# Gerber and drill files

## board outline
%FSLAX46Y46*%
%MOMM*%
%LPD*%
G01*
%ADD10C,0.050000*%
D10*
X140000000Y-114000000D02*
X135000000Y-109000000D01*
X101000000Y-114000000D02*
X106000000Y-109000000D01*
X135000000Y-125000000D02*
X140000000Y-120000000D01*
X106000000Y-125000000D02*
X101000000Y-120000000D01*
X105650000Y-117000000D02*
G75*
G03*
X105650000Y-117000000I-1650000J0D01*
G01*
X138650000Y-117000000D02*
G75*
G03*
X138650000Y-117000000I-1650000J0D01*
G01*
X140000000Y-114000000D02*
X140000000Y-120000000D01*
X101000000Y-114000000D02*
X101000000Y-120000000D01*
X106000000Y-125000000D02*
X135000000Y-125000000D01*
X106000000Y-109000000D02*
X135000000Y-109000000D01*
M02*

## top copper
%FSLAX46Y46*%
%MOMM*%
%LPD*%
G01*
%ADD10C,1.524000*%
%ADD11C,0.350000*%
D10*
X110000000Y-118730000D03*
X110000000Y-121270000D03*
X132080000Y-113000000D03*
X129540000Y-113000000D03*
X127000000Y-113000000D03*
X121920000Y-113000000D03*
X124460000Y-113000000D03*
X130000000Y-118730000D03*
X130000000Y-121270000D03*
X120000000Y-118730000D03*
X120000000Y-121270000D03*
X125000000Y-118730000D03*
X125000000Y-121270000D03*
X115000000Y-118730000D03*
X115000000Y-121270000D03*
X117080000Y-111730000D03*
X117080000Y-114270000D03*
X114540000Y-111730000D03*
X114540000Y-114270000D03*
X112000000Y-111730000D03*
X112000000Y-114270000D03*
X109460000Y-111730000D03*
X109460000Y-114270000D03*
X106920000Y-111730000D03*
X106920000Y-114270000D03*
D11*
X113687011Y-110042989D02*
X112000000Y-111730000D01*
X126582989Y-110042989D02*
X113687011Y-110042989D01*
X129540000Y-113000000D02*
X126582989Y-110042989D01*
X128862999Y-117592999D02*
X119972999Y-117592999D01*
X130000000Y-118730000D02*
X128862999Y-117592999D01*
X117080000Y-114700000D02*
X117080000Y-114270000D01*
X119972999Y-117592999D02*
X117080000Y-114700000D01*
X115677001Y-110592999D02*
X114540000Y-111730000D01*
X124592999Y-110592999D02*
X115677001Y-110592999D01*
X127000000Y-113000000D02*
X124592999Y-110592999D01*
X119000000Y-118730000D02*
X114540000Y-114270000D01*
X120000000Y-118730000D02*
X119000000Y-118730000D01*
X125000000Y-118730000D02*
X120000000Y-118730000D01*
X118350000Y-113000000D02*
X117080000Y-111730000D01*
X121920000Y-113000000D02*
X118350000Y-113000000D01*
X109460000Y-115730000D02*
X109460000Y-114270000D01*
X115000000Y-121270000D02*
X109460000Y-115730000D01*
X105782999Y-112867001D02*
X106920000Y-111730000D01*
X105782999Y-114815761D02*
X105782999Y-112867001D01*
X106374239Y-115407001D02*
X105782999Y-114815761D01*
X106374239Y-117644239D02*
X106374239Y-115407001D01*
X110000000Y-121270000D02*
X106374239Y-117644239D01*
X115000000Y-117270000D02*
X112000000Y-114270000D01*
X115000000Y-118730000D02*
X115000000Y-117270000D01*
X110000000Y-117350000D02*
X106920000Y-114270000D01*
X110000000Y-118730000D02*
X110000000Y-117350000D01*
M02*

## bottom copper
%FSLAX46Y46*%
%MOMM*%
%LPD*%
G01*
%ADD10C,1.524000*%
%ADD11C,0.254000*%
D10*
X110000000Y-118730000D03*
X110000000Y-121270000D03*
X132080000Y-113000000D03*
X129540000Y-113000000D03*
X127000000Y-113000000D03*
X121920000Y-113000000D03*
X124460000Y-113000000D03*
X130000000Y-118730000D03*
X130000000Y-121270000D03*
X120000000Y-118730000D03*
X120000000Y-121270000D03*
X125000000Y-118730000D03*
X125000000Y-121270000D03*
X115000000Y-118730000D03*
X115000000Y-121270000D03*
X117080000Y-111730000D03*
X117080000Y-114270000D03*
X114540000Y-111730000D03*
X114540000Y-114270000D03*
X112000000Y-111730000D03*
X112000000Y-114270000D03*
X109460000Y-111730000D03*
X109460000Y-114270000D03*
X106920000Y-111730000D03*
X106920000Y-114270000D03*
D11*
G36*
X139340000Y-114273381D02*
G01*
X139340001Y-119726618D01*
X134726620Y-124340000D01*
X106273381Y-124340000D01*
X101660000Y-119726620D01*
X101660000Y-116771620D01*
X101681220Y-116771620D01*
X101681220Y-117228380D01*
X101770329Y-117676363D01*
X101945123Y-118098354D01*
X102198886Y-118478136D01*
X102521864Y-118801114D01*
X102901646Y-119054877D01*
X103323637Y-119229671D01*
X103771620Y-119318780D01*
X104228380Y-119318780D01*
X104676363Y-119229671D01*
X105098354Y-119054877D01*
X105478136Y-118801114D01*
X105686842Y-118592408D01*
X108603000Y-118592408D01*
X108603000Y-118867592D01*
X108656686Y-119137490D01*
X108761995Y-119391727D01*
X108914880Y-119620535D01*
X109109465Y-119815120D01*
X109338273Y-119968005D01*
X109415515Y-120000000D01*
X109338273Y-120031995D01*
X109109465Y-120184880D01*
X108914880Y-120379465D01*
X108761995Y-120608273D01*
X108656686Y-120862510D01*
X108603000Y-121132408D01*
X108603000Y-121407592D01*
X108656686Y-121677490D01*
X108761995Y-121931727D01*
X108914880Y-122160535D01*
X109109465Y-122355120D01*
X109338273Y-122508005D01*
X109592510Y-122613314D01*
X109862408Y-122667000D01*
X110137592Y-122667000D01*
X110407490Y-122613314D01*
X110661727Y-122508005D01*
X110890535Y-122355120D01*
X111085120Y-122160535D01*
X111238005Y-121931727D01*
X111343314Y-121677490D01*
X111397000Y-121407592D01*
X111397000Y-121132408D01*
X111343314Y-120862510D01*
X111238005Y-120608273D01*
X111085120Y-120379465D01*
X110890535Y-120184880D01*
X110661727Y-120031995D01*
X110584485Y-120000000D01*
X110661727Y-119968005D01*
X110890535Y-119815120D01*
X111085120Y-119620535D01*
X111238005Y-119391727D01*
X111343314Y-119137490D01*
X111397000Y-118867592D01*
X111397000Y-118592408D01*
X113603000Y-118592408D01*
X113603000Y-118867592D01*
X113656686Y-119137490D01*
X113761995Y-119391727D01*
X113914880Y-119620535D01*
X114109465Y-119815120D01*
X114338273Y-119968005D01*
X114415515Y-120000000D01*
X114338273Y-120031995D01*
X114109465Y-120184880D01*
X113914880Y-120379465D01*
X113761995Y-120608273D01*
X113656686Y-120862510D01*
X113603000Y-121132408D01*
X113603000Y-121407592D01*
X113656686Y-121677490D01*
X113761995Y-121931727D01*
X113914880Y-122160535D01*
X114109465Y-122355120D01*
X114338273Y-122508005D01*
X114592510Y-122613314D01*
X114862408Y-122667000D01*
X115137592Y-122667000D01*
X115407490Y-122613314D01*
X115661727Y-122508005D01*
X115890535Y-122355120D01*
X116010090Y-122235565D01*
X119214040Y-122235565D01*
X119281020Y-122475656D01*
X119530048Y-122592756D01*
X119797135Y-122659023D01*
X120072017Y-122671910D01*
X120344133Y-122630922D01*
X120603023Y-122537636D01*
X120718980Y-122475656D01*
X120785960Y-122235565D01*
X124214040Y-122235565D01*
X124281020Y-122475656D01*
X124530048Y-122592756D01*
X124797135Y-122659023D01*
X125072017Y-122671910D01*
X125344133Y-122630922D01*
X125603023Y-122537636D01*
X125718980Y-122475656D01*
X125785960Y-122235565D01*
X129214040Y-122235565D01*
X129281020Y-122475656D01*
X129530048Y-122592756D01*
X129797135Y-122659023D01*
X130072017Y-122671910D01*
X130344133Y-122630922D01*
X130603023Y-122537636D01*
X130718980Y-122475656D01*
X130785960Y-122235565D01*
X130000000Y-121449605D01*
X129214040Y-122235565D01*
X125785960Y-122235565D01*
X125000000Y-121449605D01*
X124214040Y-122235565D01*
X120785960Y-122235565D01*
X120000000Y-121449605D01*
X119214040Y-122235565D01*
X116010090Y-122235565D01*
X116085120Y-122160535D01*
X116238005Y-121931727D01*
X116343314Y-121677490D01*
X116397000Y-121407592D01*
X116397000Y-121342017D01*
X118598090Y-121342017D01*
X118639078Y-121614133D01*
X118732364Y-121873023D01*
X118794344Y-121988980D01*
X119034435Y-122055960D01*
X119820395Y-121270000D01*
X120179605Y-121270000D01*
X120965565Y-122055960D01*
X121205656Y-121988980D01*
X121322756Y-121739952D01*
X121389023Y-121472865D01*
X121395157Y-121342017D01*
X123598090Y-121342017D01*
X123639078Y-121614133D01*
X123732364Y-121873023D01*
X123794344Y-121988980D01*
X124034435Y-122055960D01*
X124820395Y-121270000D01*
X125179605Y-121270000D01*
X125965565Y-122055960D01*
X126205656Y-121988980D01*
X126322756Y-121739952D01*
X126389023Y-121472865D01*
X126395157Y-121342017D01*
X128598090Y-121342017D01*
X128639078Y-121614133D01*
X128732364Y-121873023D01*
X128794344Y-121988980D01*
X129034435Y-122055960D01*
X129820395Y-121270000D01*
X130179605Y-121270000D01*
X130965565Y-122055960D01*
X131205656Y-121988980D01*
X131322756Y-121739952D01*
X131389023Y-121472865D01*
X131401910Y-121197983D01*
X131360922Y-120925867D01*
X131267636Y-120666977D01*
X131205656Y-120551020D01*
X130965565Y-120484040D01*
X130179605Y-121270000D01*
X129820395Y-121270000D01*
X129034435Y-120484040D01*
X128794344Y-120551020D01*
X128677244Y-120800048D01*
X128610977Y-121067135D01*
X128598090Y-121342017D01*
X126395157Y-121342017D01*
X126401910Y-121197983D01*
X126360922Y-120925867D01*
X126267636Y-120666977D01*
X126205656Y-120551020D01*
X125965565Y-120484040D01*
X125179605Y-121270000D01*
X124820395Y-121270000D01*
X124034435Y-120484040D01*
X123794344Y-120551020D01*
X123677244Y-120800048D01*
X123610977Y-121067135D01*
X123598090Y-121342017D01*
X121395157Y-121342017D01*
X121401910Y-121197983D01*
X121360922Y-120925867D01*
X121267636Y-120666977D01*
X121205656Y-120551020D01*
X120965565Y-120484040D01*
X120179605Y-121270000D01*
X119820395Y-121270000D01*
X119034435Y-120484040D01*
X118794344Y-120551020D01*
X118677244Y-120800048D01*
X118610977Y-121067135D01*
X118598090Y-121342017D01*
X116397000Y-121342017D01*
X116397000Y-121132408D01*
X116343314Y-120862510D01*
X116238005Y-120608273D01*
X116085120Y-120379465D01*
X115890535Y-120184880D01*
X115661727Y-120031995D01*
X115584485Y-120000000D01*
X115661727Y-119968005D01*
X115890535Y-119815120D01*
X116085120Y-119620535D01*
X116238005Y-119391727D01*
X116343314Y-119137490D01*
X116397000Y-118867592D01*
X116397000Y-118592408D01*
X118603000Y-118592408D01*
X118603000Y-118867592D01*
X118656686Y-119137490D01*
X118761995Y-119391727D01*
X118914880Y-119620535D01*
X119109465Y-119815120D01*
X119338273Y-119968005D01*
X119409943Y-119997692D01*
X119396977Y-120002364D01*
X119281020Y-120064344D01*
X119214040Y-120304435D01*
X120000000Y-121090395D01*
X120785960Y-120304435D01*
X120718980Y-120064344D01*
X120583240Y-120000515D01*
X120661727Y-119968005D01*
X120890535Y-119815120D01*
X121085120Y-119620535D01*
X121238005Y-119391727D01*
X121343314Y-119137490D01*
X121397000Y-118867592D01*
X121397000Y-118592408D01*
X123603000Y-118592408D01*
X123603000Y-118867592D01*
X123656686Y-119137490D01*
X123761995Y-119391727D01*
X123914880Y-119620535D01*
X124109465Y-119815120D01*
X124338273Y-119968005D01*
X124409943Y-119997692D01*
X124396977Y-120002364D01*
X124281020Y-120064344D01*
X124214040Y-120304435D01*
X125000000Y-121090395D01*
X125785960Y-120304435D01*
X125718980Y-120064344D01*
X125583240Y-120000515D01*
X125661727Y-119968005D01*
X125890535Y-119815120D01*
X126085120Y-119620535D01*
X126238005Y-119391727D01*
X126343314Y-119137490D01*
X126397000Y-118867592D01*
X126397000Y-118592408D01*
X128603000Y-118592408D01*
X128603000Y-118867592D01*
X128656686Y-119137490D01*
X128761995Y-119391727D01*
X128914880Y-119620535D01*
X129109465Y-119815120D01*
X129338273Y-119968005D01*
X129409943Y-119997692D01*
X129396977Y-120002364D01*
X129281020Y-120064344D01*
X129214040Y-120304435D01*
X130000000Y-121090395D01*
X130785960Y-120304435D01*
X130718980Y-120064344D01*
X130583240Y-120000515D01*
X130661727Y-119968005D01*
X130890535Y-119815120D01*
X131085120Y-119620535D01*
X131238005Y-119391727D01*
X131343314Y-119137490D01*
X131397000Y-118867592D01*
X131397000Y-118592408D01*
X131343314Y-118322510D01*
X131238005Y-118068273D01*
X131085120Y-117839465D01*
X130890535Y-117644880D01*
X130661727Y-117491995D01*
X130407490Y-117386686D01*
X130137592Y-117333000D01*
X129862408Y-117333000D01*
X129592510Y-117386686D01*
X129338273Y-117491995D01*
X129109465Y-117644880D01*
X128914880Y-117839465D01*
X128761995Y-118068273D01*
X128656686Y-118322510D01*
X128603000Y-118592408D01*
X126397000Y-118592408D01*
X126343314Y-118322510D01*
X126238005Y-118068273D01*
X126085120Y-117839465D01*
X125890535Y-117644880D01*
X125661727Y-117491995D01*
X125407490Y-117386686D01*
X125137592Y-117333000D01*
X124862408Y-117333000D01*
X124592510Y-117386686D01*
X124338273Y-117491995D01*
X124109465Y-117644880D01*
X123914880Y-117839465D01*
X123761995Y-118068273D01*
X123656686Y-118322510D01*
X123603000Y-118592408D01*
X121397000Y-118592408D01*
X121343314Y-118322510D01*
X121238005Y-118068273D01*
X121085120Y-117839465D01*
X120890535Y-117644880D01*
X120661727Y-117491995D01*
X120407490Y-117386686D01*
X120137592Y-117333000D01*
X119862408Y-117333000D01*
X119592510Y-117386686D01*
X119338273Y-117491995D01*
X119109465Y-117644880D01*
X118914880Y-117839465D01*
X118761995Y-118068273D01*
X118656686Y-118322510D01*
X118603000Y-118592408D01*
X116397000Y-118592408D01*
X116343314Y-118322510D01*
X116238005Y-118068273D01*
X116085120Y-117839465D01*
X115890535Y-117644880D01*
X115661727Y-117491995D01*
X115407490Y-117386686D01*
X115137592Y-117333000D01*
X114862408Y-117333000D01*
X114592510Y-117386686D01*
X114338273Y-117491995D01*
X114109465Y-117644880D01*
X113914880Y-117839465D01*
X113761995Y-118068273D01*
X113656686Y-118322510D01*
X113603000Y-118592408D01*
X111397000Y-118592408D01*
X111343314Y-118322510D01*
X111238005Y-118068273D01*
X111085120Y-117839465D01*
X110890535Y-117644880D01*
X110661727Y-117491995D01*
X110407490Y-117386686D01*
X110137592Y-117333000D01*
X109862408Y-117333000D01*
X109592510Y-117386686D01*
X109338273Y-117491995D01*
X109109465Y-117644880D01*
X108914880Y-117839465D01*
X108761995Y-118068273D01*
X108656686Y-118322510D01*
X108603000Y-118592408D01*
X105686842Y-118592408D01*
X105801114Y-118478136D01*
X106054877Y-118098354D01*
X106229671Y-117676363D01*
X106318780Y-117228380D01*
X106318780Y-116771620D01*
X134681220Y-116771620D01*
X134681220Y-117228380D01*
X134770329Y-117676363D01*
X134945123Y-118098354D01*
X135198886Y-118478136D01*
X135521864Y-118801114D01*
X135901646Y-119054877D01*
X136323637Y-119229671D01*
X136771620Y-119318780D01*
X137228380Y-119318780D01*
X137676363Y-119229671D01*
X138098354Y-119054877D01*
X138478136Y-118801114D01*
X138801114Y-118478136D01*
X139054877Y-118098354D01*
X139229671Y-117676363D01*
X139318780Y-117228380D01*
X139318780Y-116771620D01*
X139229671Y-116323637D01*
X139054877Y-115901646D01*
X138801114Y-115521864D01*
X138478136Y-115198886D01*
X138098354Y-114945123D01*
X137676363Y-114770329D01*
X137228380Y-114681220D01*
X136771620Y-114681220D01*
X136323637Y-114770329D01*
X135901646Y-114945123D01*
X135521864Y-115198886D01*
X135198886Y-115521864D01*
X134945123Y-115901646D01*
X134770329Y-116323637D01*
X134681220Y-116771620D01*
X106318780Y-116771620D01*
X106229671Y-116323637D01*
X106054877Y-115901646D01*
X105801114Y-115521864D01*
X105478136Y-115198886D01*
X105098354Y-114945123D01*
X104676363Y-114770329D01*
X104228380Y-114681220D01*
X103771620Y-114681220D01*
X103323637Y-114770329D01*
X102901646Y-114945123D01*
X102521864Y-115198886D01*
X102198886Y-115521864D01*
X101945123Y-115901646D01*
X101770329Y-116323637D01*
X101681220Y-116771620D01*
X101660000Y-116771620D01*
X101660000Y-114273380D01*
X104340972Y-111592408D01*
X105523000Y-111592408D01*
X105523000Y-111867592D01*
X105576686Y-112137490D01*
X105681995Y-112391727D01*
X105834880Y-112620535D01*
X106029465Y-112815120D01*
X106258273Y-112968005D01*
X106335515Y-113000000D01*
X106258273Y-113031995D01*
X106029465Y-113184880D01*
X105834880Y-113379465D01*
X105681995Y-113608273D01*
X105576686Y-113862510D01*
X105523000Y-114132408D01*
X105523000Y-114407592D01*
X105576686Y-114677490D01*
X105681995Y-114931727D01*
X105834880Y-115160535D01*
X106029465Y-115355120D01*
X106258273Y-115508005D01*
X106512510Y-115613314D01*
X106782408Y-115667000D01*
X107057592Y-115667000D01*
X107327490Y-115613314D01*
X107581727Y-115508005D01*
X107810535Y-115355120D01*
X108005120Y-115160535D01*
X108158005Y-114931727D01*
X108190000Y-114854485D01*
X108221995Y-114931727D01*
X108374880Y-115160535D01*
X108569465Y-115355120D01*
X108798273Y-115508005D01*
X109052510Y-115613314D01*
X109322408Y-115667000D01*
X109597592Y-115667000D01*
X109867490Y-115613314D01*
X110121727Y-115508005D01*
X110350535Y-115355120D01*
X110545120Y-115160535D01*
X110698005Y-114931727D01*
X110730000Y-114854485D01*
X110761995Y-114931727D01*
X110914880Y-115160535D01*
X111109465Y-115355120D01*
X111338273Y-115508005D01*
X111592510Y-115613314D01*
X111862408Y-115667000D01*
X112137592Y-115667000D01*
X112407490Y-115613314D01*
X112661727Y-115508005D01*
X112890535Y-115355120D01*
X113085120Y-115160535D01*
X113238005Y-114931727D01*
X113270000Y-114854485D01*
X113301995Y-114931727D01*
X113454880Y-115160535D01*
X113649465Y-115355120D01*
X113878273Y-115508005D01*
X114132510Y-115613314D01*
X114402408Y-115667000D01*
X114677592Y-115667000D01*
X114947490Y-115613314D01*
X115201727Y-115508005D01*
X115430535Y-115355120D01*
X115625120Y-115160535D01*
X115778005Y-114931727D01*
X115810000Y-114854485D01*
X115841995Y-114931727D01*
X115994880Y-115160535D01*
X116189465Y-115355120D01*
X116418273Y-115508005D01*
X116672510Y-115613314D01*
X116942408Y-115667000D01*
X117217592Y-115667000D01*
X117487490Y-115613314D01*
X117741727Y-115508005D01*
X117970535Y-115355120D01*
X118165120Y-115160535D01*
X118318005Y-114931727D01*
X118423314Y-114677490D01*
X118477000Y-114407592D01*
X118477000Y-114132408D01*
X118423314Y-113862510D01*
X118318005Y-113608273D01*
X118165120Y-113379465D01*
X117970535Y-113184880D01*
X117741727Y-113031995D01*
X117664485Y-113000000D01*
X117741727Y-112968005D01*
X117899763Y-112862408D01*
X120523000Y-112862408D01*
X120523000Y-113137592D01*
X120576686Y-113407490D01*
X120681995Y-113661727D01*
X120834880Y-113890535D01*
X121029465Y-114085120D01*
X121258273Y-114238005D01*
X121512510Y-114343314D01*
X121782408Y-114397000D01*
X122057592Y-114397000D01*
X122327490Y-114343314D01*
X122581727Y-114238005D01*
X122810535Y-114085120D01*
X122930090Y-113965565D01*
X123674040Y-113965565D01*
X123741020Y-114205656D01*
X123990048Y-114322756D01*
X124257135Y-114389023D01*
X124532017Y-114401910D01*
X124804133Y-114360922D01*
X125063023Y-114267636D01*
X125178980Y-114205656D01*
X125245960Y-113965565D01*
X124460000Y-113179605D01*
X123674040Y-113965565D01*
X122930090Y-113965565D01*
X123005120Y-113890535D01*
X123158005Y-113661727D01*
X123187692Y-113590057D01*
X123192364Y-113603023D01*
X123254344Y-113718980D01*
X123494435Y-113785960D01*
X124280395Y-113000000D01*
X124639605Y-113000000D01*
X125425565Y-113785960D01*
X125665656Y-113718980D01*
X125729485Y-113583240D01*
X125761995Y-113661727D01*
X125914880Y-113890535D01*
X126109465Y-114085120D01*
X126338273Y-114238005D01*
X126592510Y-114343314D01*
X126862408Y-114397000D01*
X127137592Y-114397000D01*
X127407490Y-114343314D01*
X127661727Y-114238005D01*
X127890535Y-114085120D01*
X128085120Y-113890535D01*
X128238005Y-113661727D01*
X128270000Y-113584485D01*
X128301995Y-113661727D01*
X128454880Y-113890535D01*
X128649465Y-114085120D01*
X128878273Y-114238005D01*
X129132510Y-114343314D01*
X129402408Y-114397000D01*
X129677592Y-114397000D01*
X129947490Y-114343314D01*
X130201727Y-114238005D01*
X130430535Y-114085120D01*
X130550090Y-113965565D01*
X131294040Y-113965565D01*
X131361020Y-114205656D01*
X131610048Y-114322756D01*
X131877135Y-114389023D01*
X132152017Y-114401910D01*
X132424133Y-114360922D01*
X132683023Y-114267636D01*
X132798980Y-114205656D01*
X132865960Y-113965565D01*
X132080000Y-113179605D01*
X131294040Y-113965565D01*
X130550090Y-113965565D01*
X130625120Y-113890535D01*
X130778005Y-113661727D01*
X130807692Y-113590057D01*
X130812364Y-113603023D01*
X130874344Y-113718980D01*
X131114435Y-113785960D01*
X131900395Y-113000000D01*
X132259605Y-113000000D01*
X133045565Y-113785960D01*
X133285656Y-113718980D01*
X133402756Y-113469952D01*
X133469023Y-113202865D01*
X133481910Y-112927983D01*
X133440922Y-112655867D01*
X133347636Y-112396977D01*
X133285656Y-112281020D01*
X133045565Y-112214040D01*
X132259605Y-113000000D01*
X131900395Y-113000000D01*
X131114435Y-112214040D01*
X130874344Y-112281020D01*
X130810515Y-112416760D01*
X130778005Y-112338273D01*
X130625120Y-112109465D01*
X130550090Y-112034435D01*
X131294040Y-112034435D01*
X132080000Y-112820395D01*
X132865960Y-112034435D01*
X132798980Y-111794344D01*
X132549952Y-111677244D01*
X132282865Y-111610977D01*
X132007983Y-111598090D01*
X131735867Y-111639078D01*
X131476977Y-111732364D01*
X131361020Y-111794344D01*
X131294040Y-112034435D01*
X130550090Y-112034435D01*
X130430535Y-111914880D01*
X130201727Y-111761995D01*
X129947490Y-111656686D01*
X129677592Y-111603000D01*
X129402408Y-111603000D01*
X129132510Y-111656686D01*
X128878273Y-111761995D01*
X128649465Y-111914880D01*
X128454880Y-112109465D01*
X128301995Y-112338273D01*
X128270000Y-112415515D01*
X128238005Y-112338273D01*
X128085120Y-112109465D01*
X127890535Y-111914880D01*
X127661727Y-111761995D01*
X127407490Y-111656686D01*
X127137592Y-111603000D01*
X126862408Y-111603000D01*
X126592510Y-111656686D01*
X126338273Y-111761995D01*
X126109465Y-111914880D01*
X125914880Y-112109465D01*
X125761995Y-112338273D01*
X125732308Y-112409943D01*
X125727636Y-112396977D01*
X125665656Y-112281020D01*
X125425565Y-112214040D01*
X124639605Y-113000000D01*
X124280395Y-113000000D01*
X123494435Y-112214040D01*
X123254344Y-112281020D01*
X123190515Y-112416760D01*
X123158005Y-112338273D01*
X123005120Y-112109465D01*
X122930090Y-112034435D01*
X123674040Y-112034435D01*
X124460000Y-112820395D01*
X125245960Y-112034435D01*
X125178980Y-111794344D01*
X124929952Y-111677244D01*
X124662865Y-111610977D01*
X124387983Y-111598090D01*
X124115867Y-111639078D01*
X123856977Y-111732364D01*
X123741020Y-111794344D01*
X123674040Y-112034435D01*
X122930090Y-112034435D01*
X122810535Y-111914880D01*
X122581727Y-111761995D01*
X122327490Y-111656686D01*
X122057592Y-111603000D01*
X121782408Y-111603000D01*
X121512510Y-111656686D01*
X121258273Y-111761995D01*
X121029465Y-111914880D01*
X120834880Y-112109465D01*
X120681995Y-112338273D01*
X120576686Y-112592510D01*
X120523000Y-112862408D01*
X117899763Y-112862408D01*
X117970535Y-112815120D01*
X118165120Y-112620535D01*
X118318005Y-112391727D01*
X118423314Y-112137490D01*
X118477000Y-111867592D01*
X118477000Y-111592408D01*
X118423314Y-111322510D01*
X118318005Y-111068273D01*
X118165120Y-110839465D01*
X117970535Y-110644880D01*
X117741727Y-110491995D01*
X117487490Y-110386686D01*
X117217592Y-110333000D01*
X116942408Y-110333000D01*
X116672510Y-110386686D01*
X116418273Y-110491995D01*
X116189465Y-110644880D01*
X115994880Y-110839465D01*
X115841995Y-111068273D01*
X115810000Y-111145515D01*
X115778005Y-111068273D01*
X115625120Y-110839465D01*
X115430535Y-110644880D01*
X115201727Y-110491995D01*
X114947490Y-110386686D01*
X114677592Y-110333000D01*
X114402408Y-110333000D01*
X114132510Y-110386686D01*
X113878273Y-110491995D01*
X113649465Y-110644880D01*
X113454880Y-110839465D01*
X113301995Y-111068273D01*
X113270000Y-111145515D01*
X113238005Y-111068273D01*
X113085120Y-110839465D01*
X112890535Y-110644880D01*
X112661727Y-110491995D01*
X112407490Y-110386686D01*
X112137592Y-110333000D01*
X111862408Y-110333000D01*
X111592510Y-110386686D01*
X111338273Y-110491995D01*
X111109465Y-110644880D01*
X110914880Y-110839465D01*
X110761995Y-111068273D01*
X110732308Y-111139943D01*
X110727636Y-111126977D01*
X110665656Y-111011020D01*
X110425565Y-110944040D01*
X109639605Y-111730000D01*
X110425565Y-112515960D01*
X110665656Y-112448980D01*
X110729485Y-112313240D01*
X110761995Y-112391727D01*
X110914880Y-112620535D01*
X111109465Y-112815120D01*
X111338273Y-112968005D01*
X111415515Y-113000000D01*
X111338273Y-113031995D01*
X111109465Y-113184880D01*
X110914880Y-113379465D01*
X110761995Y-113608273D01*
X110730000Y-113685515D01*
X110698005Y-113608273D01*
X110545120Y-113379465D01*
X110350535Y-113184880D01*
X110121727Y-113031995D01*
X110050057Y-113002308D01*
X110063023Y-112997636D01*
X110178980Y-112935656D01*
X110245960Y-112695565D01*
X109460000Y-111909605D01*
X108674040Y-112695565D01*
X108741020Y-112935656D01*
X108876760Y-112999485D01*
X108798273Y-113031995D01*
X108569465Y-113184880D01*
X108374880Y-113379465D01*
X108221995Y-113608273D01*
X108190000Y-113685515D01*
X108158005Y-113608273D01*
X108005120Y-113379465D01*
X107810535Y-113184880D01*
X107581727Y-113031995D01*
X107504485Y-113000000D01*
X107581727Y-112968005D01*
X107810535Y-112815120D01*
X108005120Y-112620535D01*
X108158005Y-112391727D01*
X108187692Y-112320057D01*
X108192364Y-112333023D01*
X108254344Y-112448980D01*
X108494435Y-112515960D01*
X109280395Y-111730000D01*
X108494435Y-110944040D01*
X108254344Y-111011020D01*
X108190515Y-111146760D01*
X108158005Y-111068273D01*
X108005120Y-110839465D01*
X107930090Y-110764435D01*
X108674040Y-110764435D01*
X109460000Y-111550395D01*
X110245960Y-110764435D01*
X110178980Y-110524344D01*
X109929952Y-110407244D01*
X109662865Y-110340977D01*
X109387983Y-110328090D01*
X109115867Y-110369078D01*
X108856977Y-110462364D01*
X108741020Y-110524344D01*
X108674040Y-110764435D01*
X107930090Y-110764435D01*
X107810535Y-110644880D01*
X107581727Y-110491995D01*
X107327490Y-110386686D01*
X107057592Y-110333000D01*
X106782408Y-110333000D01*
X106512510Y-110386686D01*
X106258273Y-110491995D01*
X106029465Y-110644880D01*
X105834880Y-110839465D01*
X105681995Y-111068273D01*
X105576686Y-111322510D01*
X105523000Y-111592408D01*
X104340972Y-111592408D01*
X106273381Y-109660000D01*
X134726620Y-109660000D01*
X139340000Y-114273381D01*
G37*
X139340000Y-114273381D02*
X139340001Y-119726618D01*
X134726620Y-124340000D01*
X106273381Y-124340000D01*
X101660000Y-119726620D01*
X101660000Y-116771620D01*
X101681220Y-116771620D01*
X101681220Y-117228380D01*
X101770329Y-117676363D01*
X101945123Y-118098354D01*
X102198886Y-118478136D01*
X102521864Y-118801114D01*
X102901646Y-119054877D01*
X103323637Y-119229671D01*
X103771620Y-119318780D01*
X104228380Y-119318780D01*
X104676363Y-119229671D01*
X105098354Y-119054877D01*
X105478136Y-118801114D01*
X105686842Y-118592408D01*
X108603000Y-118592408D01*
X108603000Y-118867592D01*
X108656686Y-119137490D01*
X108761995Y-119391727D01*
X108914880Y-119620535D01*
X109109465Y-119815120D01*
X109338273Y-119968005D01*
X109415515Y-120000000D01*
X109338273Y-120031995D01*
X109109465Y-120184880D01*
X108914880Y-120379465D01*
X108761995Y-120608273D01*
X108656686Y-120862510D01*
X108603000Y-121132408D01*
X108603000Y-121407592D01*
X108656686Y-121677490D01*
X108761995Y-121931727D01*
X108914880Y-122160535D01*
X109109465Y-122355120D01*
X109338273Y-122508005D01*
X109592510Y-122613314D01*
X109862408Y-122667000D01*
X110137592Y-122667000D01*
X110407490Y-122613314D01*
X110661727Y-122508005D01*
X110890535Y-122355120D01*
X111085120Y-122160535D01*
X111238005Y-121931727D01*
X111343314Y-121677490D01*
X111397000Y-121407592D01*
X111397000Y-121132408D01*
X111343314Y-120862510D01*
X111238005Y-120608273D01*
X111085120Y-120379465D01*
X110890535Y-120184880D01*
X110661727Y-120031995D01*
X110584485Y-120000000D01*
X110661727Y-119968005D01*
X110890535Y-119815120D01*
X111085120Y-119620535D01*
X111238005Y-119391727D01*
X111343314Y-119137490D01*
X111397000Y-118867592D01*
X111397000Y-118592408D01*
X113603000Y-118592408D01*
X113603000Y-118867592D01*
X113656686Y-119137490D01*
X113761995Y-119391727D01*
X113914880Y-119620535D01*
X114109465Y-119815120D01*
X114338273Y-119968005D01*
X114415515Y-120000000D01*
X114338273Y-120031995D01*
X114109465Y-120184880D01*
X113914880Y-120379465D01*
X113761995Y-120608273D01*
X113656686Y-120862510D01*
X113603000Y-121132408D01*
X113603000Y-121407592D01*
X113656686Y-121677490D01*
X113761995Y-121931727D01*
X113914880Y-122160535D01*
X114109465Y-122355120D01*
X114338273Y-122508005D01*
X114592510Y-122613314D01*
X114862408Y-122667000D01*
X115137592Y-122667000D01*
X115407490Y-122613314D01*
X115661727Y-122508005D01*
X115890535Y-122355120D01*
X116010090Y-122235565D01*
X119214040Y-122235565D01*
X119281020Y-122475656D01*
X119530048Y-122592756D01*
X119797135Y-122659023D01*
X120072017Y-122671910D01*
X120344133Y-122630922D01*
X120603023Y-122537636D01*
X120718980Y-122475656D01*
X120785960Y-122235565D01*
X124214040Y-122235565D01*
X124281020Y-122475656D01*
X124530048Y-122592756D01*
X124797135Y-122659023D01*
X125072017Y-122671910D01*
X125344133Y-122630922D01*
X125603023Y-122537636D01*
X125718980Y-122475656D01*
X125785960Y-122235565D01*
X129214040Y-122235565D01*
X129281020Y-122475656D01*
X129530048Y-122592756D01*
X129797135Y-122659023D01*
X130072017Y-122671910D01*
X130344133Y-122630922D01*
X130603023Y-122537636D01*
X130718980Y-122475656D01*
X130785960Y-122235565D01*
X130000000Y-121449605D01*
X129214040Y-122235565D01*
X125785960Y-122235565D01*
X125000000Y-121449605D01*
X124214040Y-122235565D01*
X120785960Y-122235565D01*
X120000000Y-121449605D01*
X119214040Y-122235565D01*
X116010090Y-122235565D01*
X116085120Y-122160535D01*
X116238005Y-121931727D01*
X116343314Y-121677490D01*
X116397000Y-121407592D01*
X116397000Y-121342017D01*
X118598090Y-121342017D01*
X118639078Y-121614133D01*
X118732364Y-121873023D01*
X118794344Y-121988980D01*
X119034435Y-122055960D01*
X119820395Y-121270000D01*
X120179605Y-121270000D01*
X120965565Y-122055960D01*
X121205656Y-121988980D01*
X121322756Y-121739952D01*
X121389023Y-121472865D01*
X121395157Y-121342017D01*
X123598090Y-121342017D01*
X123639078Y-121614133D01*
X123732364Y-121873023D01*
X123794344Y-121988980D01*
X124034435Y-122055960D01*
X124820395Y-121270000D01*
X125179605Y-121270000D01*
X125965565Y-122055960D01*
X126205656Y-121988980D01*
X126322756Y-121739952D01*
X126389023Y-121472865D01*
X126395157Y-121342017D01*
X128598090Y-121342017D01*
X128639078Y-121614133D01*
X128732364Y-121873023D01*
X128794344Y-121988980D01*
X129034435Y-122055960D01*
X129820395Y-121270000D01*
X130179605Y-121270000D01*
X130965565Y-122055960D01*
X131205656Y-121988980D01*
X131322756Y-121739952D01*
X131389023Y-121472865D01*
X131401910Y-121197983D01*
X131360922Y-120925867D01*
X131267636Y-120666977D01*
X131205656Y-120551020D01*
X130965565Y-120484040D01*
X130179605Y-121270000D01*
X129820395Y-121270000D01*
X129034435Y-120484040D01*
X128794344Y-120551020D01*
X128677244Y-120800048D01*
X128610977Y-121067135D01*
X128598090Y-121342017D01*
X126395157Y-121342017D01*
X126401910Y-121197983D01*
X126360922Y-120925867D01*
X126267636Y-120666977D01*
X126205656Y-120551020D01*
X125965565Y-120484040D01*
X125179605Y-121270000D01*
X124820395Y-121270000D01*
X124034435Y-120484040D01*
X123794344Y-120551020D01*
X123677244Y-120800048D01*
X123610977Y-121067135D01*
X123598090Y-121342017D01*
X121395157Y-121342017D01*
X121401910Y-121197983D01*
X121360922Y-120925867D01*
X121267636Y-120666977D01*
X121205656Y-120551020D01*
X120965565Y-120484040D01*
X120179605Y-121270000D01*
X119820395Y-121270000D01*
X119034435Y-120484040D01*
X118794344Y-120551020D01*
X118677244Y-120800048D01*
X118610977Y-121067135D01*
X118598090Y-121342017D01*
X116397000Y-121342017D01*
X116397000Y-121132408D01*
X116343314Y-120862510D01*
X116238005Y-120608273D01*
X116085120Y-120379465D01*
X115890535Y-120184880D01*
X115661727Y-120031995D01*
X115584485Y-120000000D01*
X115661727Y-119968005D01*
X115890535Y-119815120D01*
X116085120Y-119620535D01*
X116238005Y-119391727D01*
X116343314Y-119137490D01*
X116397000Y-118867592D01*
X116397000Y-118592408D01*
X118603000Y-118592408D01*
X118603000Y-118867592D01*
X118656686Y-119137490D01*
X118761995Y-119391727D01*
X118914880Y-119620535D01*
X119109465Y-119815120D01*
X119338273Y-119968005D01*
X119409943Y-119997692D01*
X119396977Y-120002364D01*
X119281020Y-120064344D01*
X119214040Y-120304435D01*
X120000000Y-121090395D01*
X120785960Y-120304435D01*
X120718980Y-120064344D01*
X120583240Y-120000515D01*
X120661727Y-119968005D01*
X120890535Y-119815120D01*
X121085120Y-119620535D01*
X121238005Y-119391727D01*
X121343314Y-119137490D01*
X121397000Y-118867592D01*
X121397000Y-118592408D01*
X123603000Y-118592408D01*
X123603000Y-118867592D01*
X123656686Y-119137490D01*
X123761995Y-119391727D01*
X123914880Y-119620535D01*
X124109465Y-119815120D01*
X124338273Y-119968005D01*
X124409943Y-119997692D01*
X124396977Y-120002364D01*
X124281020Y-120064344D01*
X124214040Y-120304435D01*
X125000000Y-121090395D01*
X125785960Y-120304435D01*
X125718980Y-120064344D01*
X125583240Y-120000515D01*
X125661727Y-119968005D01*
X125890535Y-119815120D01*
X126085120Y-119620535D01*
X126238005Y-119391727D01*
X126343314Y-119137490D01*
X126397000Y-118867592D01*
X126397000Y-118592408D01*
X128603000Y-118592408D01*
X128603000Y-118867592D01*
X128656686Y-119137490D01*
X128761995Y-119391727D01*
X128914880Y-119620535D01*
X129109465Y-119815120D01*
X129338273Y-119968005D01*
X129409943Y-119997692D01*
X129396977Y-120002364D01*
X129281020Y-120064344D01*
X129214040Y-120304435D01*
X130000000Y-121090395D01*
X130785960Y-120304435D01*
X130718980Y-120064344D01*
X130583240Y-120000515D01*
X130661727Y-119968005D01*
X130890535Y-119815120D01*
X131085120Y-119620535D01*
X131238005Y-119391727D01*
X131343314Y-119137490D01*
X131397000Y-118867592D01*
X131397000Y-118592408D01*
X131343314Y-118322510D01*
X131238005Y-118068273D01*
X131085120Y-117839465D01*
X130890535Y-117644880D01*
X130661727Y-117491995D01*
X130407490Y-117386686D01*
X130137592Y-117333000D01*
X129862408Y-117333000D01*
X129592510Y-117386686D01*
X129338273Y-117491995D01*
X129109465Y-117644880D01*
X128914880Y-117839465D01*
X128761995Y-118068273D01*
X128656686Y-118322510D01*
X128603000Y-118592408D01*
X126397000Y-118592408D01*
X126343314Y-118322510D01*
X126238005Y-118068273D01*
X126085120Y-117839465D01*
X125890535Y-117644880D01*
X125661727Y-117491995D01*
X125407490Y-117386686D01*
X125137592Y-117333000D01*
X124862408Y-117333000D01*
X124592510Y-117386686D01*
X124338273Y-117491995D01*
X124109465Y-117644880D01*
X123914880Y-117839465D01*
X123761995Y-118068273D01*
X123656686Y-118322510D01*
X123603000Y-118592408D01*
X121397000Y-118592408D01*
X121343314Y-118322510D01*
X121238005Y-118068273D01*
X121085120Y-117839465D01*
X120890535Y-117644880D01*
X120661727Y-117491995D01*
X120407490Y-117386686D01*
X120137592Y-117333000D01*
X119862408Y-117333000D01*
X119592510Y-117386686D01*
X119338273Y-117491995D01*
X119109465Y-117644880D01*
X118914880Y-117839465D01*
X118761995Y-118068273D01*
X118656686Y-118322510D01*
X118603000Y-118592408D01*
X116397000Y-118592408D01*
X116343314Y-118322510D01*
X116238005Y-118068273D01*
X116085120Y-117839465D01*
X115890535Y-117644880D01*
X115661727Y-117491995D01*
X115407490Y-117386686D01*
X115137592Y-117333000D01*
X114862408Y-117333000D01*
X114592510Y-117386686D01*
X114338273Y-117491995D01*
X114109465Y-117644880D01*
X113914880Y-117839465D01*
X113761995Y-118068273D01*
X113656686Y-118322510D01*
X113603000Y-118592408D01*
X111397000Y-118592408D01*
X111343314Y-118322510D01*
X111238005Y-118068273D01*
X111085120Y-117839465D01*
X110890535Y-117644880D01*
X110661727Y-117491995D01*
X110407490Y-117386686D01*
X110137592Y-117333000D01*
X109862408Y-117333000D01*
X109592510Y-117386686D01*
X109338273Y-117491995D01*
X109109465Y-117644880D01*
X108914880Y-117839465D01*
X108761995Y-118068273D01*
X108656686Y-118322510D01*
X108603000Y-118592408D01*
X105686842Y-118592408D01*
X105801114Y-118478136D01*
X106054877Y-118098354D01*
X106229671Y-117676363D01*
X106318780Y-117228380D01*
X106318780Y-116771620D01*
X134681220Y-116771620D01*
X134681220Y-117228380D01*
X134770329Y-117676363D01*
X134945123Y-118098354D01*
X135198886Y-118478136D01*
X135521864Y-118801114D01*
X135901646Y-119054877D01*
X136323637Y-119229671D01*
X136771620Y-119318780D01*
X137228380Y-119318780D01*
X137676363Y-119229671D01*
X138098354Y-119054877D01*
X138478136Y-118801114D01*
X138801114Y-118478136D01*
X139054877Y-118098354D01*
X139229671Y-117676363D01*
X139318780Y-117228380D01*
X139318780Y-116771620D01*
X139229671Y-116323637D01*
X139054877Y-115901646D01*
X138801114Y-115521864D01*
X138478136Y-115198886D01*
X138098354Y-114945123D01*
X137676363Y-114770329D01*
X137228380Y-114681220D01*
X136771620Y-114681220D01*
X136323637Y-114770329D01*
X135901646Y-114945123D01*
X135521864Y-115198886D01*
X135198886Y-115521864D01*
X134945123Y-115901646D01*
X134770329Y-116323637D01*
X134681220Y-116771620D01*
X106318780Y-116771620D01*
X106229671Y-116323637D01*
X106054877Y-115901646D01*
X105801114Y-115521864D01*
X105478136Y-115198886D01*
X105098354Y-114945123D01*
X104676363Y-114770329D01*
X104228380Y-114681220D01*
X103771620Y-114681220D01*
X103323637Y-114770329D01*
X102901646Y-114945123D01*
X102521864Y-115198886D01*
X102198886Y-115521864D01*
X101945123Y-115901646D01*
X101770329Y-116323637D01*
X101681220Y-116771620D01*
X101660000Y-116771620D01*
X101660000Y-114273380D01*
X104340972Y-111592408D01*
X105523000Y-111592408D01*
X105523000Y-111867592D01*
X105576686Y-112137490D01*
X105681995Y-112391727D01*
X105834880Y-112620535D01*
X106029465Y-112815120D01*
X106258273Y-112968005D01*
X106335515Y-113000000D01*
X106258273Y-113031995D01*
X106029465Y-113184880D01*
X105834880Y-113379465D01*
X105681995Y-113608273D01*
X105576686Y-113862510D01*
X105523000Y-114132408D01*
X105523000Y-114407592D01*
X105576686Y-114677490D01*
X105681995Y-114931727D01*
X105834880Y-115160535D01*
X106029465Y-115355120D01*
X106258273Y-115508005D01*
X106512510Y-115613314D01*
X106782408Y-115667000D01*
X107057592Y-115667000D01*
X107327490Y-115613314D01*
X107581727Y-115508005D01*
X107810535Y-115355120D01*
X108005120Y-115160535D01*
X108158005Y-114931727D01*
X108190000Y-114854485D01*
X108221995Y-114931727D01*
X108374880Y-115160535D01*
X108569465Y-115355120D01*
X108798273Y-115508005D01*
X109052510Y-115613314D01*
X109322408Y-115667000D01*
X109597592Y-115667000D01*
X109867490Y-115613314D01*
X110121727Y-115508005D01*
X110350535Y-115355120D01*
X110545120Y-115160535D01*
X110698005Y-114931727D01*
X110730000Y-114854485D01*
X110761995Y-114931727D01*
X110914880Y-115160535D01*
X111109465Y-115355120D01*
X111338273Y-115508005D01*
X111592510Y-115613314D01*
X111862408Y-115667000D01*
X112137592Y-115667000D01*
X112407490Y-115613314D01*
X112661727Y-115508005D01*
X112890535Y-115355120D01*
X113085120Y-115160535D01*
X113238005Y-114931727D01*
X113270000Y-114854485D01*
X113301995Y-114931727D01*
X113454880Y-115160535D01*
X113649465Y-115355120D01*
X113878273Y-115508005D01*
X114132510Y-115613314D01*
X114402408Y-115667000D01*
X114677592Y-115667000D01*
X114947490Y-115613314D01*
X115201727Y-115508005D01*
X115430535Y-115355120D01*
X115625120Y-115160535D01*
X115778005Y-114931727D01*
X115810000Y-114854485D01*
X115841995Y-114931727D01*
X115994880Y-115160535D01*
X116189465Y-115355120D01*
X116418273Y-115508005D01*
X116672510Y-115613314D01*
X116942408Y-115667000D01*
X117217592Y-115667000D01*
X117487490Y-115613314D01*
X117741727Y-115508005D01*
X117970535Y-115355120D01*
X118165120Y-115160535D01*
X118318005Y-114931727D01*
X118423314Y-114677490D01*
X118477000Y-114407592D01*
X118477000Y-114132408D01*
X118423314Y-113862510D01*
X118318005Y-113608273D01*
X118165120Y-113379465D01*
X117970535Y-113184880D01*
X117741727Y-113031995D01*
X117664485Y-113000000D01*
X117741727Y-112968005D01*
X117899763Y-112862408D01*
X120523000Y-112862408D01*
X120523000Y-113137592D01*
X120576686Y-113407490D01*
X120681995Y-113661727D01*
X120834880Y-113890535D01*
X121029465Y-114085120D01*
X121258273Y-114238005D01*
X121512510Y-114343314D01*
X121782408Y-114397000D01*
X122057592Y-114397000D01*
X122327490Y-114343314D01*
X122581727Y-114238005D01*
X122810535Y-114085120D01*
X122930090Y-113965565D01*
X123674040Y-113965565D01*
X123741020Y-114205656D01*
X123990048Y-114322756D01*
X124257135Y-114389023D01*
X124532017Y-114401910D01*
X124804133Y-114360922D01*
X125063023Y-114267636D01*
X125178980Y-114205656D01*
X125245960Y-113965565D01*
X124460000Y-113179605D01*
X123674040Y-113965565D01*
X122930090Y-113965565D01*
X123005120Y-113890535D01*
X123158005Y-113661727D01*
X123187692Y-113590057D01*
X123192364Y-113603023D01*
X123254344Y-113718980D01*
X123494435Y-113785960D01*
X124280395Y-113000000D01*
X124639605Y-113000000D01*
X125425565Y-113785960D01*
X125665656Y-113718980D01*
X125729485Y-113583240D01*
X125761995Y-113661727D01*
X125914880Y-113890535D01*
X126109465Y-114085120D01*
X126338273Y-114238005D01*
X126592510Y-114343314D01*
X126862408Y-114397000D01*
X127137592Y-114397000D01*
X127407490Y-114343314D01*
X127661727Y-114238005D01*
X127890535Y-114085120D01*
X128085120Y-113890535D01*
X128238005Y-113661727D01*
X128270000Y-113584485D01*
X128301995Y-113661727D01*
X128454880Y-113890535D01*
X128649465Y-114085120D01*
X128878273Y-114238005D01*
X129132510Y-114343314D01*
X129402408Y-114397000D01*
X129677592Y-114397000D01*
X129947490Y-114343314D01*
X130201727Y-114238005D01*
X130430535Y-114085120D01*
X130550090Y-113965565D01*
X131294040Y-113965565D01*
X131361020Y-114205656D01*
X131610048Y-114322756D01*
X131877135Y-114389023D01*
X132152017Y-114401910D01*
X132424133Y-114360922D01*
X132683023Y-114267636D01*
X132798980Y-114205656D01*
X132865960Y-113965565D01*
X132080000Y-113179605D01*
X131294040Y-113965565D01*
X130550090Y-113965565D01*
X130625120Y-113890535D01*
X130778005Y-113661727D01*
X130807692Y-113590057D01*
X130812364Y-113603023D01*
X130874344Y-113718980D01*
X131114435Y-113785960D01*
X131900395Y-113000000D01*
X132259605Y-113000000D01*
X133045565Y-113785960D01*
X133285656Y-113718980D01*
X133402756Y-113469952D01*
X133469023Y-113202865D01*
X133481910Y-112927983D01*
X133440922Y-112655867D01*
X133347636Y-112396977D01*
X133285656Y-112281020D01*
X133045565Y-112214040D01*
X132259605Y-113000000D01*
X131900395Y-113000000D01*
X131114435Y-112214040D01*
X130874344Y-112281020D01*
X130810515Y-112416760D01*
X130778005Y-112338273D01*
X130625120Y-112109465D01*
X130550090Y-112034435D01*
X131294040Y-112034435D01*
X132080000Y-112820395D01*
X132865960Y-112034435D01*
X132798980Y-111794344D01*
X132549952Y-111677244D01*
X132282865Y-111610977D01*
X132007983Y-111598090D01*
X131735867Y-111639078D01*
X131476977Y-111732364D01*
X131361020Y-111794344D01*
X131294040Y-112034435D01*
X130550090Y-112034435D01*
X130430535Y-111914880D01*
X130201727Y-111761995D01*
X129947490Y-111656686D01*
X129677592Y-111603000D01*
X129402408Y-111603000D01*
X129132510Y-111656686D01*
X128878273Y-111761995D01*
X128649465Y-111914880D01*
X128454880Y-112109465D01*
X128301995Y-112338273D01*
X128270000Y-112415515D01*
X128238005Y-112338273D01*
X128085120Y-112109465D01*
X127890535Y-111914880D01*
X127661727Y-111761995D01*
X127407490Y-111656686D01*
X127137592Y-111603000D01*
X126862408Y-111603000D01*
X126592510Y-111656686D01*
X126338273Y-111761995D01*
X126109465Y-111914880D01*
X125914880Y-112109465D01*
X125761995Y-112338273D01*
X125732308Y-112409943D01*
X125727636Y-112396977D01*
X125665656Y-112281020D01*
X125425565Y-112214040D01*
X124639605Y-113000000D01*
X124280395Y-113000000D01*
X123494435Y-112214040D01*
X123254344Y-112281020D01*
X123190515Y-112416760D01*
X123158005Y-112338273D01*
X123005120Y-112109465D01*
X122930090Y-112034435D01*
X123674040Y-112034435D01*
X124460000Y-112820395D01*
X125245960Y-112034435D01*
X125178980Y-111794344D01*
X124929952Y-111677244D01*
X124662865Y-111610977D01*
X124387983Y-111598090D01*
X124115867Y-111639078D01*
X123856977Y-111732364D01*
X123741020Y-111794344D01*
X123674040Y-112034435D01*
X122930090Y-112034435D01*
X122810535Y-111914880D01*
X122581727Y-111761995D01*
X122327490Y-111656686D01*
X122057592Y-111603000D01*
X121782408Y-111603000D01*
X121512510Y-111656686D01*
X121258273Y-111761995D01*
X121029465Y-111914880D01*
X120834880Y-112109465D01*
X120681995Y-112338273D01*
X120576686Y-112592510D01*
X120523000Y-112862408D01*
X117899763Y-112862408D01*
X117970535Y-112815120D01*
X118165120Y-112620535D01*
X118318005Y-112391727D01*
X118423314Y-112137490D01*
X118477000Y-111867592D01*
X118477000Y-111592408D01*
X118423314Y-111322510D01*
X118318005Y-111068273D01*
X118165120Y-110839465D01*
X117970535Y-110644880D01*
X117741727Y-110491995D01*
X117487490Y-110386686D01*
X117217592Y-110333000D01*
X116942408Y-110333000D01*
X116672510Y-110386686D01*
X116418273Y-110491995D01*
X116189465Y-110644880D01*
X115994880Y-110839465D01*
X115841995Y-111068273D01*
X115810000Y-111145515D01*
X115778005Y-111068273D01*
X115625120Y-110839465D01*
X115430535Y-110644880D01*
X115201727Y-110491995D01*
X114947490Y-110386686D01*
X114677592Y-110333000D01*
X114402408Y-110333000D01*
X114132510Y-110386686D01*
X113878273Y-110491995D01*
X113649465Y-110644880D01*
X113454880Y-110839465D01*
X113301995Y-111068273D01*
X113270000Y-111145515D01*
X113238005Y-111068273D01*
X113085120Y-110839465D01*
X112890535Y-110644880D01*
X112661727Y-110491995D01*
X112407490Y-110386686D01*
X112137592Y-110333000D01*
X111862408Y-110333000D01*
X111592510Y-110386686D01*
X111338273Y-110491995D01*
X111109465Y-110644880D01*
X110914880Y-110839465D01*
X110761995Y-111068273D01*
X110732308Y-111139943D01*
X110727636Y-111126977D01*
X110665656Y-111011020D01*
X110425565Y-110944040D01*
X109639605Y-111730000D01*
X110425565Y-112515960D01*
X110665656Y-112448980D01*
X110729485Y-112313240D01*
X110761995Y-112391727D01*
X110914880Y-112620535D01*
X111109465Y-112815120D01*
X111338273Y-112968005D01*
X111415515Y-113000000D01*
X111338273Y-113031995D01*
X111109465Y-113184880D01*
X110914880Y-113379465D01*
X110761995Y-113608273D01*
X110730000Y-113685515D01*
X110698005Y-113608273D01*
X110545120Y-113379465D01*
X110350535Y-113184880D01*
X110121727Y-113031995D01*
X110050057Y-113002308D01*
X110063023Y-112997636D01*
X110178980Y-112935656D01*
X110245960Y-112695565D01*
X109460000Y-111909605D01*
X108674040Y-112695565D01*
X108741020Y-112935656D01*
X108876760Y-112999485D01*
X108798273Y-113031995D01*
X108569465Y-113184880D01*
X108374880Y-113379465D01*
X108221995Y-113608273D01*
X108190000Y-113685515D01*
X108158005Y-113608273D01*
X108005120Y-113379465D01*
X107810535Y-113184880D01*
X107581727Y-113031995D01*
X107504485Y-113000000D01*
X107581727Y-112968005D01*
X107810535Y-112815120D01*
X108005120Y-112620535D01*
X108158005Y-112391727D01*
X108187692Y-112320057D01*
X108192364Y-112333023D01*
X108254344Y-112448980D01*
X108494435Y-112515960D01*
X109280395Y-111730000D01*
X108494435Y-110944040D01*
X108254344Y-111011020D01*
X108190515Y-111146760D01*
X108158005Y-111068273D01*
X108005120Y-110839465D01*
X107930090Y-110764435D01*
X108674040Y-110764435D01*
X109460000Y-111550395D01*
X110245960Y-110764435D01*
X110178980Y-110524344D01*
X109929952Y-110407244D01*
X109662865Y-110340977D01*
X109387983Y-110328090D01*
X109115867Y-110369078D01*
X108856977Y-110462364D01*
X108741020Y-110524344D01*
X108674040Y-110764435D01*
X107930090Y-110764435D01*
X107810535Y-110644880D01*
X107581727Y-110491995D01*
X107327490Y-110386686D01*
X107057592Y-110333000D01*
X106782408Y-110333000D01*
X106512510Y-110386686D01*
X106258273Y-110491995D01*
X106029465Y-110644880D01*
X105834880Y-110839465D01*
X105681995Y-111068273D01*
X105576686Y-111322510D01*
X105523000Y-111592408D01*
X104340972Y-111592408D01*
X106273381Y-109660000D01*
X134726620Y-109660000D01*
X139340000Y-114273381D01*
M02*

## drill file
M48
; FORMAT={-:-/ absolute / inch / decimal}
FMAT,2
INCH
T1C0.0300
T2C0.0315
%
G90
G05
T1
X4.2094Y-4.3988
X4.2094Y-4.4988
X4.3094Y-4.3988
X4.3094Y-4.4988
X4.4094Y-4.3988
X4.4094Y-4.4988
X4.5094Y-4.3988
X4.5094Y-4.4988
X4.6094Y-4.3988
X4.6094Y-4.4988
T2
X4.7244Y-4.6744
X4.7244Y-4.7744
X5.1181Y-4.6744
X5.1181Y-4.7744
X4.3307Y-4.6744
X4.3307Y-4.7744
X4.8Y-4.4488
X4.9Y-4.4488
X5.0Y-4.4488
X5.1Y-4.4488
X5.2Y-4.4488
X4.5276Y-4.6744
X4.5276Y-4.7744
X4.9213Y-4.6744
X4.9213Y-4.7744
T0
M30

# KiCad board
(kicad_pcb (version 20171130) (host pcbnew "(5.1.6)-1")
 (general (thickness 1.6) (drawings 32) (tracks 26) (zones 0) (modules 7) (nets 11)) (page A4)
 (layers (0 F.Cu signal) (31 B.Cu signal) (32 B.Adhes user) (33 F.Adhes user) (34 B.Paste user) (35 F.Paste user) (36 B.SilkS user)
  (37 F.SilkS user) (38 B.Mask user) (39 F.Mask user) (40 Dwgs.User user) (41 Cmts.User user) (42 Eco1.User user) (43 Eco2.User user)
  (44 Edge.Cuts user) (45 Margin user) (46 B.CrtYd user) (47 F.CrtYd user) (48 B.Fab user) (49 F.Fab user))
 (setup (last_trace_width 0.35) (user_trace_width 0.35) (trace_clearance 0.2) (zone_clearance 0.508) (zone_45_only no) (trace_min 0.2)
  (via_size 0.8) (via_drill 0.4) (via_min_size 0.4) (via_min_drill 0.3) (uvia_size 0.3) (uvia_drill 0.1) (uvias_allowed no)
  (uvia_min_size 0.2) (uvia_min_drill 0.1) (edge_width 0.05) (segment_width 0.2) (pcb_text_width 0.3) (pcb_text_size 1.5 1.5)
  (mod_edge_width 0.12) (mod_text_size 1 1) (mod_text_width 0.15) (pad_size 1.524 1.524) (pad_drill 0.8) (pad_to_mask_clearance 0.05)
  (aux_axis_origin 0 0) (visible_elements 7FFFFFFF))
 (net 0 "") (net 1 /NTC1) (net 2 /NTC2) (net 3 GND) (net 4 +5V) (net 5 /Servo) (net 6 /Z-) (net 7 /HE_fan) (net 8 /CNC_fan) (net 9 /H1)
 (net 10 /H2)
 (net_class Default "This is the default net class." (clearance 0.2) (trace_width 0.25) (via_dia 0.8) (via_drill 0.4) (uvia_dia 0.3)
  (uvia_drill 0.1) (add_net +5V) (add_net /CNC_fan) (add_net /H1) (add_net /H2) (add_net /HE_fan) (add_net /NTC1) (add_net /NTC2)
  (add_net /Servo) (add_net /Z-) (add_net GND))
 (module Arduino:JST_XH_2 (layer F.Cu) (at 110 120 270)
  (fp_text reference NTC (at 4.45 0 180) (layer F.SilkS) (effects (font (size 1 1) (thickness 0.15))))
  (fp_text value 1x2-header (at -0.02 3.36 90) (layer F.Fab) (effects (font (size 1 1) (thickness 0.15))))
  (pad 1 thru_hole circle (at -1.27 0 270) (size 1.524 1.524) (drill 0.8) (layers *.Cu *.Mask) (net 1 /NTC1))
  (pad 2 thru_hole circle (at 1.27 0 270) (size 1.524 1.524) (drill 0.8) (layers *.Cu *.Mask) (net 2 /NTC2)))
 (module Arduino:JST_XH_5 (layer F.Cu) (at 127 113)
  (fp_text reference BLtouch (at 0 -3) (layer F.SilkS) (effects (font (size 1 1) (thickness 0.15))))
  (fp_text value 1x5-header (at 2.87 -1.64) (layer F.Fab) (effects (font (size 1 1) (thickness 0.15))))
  (pad 5 thru_hole circle (at 5.08 0) (size 1.524 1.524) (drill 0.8) (layers *.Cu *.Mask) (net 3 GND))
  (pad 4 thru_hole circle (at 2.54 0) (size 1.524 1.524) (drill 0.8) (layers *.Cu *.Mask) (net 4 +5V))
  (pad 3 thru_hole circle (at 0 0) (size 1.524 1.524) (drill 0.8) (layers *.Cu *.Mask) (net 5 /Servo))
  (pad 1 thru_hole circle (at -5.08 0) (size 1.524 1.524) (drill 0.8) (layers *.Cu *.Mask) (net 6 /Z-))
  (pad 2 thru_hole circle (at -2.54 0) (size 1.524 1.524) (drill 0.8) (layers *.Cu *.Mask) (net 3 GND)))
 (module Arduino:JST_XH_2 (layer F.Cu) (at 130 120 270)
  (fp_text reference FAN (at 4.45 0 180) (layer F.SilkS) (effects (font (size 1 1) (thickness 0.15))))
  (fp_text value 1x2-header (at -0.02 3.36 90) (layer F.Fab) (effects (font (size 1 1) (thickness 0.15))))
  (pad 1 thru_hole circle (at -1.27 0 270) (size 1.524 1.524) (drill 0.8) (layers *.Cu *.Mask) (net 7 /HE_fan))
  (pad 2 thru_hole circle (at 1.27 0 270) (size 1.524 1.524) (drill 0.8) (layers *.Cu *.Mask) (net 3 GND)))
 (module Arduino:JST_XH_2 (layer F.Cu) (at 120 120 270)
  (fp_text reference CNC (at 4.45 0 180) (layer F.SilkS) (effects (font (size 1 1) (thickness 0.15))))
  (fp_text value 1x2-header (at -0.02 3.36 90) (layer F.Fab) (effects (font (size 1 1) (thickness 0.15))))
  (pad 1 thru_hole circle (at -1.27 0 270) (size 1.524 1.524) (drill 0.8) (layers *.Cu *.Mask) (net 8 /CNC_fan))
  (pad 2 thru_hole circle (at 1.27 0 270) (size 1.524 1.524) (drill 0.8) (layers *.Cu *.Mask) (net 3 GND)))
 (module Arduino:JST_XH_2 (layer F.Cu) (at 125 120 270)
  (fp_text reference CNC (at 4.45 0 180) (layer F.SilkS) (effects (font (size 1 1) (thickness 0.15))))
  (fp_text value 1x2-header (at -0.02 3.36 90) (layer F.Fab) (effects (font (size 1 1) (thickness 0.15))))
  (pad 1 thru_hole circle (at -1.27 0 270) (size 1.524 1.524) (drill 0.8) (layers *.Cu *.Mask) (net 8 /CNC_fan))
  (pad 2 thru_hole circle (at 1.27 0 270) (size 1.524 1.524) (drill 0.8) (layers *.Cu *.Mask) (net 3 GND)))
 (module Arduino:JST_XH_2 (layer F.Cu) (at 115 120 270)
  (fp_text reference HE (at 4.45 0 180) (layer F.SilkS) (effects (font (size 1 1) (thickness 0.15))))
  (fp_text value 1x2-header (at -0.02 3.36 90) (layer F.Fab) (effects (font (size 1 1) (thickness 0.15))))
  (pad 1 thru_hole circle (at -1.27 0 270) (size 1.524 1.524) (drill 0.8) (layers *.Cu *.Mask) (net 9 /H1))
  (pad 2 thru_hole circle (at 1.27 0 270) (size 1.524 1.524) (drill 0.8) (layers *.Cu *.Mask) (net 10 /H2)))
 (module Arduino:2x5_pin (layer F.Cu) (at 112 113 90)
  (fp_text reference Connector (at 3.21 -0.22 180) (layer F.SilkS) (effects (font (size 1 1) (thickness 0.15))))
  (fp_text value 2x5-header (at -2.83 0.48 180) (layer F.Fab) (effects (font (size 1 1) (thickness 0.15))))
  (pad 10 thru_hole circle (at 1.27 5.08 90) (size 1.524 1.524) (drill 0.762) (layers *.Cu *.Mask) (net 6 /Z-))
  (pad 9 thru_hole circle (at -1.27 5.08 90) (size 1.524 1.524) (drill 0.762) (layers *.Cu *.Mask) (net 7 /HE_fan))
  (pad 8 thru_hole circle (at 1.27 2.54 90) (size 1.524 1.524) (drill 0.762) (layers *.Cu *.Mask) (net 5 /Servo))
  (pad 7 thru_hole circle (at -1.27 2.54 90) (size 1.524 1.524) (drill 0.762) (layers *.Cu *.Mask) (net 8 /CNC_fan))
  (pad 6 thru_hole circle (at 1.27 0 90) (size 1.524 1.524) (drill 0.762) (layers *.Cu *.Mask) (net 4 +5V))
  (pad 5 thru_hole circle (at -1.27 0 90) (size 1.524 1.524) (drill 0.762) (layers *.Cu *.Mask) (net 9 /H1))
  (pad 4 thru_hole circle (at 1.27 -2.54 90) (size 1.524 1.524) (drill 0.762) (layers *.Cu *.Mask) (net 3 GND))
  (pad 3 thru_hole circle (at -1.27 -2.54 90) (size 1.524 1.524) (drill 0.762) (layers *.Cu *.Mask) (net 10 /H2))
  (pad 2 thru_hole circle (at 1.27 -5.08 90) (size 1.524 1.524) (drill 0.762) (layers *.Cu *.Mask) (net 2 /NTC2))
  (pad 1 thru_hole circle (at -1.27 -5.08 90) (size 1.524 1.524) (drill 0.762) (layers *.Cu *.Mask) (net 1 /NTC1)))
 (gr_line (start 140 114) (end 135 109) (layer Edge.Cuts) (width 0.05))
 (gr_line (start 101 114) (end 106 109) (layer Edge.Cuts) (width 0.05))
 (gr_line (start 135 125) (end 140 120) (layer Edge.Cuts) (width 0.05))
 (gr_line (start 106 125) (end 101 120) (layer Edge.Cuts) (width 0.05))
 (gr_circle (center 104 117) (end 105.65 117) (layer Edge.Cuts) (width 0.05))
 (gr_circle (center 137 117) (end 138.65 117) (layer Edge.Cuts) (width 0.05))
 (gr_line (start 140 114) (end 140 120) (layer Edge.Cuts) (width 0.05))
 (gr_line (start 101 114) (end 101 120) (layer Edge.Cuts) (width 0.05))
 (gr_line (start 106 125) (end 135 125) (layer Edge.Cuts) (width 0.05))
 (gr_line (start 106 109) (end 135 109) (layer Edge.Cuts) (width 0.05))
 (segment (start 113.687011 110.042989) (end 112 111.73) (width 0.35) (layer F.Cu) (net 4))
 (segment (start 126.582989 110.042989) (end 113.687011 110.042989) (width 0.35) (layer F.Cu) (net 4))
 (segment (start 129.54 113) (end 126.582989 110.042989) (width 0.35) (layer F.Cu) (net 4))
 (segment (start 128.862999 117.592999) (end 119.972999 117.592999) (width 0.35) (layer F.Cu) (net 7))
 (segment (start 130 118.73) (end 128.862999 117.592999) (width 0.35) (layer F.Cu) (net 7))
 (segment (start 117.08 114.7) (end 117.08 114.27) (width 0.35) (layer F.Cu) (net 7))
 (segment (start 119.972999 117.592999) (end 117.08 114.7) (width 0.35) (layer F.Cu) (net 7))
 (segment (start 115.677001 110.592999) (end 114.54 111.73) (width 0.35) (layer F.Cu) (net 5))
 (segment (start 124.592999 110.592999) (end 115.677001 110.592999) (width 0.35) (layer F.Cu) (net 5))
 (segment (start 127 113) (end 124.592999 110.592999) (width 0.35) (layer F.Cu) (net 5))
 (segment (start 119 118.73) (end 114.54 114.27) (width 0.35) (layer F.Cu) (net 8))
 (segment (start 120 118.73) (end 119 118.73) (width 0.35) (layer F.Cu) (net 8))
 (segment (start 125 118.73) (end 120 118.73) (width 0.35) (layer F.Cu) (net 8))
 (segment (start 118.35 113) (end 117.08 111.73) (width 0.35) (layer F.Cu) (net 6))
 (segment (start 121.92 113) (end 118.35 113) (width 0.35) (layer F.Cu) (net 6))
 (segment (start 109.46 115.73) (end 109.46 114.27) (width 0.35) (layer F.Cu) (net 10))
 (segment (start 115 121.27) (end 109.46 115.73) (width 0.35) (layer F.Cu) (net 10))
 (segment (start 105.782999 112.867001) (end 106.92 111.73) (width 0.35) (layer F.Cu) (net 2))
 (segment (start 105.782999 114.815761) (end 105.782999 112.867001) (width 0.35) (layer F.Cu) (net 2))
 (segment (start 106.374239 115.407001) (end 105.782999 114.815761) (width 0.35) (layer F.Cu) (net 2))
 (segment (start 106.374239 117.644239) (end 106.374239 115.407001) (width 0.35) (layer F.Cu) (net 2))
 (segment (start 110 121.27) (end 106.374239 117.644239) (width 0.35) (layer F.Cu) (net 2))
 (segment (start 115 117.27) (end 112 114.27) (width 0.35) (layer F.Cu) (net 9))
 (segment (start 115 118.73) (end 115 117.27) (width 0.35) (layer F.Cu) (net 9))
 (segment (start 110 117.35) (end 106.92 114.27) (width 0.35) (layer F.Cu) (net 1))
 (segment (start 110 118.73) (end 110 117.35) (width 0.35) (layer F.Cu) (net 1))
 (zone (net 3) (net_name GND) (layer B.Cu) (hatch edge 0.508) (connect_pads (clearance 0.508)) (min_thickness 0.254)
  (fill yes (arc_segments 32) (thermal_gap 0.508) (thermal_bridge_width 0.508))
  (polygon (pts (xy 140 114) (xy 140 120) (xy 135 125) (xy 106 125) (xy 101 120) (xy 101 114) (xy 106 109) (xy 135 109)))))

